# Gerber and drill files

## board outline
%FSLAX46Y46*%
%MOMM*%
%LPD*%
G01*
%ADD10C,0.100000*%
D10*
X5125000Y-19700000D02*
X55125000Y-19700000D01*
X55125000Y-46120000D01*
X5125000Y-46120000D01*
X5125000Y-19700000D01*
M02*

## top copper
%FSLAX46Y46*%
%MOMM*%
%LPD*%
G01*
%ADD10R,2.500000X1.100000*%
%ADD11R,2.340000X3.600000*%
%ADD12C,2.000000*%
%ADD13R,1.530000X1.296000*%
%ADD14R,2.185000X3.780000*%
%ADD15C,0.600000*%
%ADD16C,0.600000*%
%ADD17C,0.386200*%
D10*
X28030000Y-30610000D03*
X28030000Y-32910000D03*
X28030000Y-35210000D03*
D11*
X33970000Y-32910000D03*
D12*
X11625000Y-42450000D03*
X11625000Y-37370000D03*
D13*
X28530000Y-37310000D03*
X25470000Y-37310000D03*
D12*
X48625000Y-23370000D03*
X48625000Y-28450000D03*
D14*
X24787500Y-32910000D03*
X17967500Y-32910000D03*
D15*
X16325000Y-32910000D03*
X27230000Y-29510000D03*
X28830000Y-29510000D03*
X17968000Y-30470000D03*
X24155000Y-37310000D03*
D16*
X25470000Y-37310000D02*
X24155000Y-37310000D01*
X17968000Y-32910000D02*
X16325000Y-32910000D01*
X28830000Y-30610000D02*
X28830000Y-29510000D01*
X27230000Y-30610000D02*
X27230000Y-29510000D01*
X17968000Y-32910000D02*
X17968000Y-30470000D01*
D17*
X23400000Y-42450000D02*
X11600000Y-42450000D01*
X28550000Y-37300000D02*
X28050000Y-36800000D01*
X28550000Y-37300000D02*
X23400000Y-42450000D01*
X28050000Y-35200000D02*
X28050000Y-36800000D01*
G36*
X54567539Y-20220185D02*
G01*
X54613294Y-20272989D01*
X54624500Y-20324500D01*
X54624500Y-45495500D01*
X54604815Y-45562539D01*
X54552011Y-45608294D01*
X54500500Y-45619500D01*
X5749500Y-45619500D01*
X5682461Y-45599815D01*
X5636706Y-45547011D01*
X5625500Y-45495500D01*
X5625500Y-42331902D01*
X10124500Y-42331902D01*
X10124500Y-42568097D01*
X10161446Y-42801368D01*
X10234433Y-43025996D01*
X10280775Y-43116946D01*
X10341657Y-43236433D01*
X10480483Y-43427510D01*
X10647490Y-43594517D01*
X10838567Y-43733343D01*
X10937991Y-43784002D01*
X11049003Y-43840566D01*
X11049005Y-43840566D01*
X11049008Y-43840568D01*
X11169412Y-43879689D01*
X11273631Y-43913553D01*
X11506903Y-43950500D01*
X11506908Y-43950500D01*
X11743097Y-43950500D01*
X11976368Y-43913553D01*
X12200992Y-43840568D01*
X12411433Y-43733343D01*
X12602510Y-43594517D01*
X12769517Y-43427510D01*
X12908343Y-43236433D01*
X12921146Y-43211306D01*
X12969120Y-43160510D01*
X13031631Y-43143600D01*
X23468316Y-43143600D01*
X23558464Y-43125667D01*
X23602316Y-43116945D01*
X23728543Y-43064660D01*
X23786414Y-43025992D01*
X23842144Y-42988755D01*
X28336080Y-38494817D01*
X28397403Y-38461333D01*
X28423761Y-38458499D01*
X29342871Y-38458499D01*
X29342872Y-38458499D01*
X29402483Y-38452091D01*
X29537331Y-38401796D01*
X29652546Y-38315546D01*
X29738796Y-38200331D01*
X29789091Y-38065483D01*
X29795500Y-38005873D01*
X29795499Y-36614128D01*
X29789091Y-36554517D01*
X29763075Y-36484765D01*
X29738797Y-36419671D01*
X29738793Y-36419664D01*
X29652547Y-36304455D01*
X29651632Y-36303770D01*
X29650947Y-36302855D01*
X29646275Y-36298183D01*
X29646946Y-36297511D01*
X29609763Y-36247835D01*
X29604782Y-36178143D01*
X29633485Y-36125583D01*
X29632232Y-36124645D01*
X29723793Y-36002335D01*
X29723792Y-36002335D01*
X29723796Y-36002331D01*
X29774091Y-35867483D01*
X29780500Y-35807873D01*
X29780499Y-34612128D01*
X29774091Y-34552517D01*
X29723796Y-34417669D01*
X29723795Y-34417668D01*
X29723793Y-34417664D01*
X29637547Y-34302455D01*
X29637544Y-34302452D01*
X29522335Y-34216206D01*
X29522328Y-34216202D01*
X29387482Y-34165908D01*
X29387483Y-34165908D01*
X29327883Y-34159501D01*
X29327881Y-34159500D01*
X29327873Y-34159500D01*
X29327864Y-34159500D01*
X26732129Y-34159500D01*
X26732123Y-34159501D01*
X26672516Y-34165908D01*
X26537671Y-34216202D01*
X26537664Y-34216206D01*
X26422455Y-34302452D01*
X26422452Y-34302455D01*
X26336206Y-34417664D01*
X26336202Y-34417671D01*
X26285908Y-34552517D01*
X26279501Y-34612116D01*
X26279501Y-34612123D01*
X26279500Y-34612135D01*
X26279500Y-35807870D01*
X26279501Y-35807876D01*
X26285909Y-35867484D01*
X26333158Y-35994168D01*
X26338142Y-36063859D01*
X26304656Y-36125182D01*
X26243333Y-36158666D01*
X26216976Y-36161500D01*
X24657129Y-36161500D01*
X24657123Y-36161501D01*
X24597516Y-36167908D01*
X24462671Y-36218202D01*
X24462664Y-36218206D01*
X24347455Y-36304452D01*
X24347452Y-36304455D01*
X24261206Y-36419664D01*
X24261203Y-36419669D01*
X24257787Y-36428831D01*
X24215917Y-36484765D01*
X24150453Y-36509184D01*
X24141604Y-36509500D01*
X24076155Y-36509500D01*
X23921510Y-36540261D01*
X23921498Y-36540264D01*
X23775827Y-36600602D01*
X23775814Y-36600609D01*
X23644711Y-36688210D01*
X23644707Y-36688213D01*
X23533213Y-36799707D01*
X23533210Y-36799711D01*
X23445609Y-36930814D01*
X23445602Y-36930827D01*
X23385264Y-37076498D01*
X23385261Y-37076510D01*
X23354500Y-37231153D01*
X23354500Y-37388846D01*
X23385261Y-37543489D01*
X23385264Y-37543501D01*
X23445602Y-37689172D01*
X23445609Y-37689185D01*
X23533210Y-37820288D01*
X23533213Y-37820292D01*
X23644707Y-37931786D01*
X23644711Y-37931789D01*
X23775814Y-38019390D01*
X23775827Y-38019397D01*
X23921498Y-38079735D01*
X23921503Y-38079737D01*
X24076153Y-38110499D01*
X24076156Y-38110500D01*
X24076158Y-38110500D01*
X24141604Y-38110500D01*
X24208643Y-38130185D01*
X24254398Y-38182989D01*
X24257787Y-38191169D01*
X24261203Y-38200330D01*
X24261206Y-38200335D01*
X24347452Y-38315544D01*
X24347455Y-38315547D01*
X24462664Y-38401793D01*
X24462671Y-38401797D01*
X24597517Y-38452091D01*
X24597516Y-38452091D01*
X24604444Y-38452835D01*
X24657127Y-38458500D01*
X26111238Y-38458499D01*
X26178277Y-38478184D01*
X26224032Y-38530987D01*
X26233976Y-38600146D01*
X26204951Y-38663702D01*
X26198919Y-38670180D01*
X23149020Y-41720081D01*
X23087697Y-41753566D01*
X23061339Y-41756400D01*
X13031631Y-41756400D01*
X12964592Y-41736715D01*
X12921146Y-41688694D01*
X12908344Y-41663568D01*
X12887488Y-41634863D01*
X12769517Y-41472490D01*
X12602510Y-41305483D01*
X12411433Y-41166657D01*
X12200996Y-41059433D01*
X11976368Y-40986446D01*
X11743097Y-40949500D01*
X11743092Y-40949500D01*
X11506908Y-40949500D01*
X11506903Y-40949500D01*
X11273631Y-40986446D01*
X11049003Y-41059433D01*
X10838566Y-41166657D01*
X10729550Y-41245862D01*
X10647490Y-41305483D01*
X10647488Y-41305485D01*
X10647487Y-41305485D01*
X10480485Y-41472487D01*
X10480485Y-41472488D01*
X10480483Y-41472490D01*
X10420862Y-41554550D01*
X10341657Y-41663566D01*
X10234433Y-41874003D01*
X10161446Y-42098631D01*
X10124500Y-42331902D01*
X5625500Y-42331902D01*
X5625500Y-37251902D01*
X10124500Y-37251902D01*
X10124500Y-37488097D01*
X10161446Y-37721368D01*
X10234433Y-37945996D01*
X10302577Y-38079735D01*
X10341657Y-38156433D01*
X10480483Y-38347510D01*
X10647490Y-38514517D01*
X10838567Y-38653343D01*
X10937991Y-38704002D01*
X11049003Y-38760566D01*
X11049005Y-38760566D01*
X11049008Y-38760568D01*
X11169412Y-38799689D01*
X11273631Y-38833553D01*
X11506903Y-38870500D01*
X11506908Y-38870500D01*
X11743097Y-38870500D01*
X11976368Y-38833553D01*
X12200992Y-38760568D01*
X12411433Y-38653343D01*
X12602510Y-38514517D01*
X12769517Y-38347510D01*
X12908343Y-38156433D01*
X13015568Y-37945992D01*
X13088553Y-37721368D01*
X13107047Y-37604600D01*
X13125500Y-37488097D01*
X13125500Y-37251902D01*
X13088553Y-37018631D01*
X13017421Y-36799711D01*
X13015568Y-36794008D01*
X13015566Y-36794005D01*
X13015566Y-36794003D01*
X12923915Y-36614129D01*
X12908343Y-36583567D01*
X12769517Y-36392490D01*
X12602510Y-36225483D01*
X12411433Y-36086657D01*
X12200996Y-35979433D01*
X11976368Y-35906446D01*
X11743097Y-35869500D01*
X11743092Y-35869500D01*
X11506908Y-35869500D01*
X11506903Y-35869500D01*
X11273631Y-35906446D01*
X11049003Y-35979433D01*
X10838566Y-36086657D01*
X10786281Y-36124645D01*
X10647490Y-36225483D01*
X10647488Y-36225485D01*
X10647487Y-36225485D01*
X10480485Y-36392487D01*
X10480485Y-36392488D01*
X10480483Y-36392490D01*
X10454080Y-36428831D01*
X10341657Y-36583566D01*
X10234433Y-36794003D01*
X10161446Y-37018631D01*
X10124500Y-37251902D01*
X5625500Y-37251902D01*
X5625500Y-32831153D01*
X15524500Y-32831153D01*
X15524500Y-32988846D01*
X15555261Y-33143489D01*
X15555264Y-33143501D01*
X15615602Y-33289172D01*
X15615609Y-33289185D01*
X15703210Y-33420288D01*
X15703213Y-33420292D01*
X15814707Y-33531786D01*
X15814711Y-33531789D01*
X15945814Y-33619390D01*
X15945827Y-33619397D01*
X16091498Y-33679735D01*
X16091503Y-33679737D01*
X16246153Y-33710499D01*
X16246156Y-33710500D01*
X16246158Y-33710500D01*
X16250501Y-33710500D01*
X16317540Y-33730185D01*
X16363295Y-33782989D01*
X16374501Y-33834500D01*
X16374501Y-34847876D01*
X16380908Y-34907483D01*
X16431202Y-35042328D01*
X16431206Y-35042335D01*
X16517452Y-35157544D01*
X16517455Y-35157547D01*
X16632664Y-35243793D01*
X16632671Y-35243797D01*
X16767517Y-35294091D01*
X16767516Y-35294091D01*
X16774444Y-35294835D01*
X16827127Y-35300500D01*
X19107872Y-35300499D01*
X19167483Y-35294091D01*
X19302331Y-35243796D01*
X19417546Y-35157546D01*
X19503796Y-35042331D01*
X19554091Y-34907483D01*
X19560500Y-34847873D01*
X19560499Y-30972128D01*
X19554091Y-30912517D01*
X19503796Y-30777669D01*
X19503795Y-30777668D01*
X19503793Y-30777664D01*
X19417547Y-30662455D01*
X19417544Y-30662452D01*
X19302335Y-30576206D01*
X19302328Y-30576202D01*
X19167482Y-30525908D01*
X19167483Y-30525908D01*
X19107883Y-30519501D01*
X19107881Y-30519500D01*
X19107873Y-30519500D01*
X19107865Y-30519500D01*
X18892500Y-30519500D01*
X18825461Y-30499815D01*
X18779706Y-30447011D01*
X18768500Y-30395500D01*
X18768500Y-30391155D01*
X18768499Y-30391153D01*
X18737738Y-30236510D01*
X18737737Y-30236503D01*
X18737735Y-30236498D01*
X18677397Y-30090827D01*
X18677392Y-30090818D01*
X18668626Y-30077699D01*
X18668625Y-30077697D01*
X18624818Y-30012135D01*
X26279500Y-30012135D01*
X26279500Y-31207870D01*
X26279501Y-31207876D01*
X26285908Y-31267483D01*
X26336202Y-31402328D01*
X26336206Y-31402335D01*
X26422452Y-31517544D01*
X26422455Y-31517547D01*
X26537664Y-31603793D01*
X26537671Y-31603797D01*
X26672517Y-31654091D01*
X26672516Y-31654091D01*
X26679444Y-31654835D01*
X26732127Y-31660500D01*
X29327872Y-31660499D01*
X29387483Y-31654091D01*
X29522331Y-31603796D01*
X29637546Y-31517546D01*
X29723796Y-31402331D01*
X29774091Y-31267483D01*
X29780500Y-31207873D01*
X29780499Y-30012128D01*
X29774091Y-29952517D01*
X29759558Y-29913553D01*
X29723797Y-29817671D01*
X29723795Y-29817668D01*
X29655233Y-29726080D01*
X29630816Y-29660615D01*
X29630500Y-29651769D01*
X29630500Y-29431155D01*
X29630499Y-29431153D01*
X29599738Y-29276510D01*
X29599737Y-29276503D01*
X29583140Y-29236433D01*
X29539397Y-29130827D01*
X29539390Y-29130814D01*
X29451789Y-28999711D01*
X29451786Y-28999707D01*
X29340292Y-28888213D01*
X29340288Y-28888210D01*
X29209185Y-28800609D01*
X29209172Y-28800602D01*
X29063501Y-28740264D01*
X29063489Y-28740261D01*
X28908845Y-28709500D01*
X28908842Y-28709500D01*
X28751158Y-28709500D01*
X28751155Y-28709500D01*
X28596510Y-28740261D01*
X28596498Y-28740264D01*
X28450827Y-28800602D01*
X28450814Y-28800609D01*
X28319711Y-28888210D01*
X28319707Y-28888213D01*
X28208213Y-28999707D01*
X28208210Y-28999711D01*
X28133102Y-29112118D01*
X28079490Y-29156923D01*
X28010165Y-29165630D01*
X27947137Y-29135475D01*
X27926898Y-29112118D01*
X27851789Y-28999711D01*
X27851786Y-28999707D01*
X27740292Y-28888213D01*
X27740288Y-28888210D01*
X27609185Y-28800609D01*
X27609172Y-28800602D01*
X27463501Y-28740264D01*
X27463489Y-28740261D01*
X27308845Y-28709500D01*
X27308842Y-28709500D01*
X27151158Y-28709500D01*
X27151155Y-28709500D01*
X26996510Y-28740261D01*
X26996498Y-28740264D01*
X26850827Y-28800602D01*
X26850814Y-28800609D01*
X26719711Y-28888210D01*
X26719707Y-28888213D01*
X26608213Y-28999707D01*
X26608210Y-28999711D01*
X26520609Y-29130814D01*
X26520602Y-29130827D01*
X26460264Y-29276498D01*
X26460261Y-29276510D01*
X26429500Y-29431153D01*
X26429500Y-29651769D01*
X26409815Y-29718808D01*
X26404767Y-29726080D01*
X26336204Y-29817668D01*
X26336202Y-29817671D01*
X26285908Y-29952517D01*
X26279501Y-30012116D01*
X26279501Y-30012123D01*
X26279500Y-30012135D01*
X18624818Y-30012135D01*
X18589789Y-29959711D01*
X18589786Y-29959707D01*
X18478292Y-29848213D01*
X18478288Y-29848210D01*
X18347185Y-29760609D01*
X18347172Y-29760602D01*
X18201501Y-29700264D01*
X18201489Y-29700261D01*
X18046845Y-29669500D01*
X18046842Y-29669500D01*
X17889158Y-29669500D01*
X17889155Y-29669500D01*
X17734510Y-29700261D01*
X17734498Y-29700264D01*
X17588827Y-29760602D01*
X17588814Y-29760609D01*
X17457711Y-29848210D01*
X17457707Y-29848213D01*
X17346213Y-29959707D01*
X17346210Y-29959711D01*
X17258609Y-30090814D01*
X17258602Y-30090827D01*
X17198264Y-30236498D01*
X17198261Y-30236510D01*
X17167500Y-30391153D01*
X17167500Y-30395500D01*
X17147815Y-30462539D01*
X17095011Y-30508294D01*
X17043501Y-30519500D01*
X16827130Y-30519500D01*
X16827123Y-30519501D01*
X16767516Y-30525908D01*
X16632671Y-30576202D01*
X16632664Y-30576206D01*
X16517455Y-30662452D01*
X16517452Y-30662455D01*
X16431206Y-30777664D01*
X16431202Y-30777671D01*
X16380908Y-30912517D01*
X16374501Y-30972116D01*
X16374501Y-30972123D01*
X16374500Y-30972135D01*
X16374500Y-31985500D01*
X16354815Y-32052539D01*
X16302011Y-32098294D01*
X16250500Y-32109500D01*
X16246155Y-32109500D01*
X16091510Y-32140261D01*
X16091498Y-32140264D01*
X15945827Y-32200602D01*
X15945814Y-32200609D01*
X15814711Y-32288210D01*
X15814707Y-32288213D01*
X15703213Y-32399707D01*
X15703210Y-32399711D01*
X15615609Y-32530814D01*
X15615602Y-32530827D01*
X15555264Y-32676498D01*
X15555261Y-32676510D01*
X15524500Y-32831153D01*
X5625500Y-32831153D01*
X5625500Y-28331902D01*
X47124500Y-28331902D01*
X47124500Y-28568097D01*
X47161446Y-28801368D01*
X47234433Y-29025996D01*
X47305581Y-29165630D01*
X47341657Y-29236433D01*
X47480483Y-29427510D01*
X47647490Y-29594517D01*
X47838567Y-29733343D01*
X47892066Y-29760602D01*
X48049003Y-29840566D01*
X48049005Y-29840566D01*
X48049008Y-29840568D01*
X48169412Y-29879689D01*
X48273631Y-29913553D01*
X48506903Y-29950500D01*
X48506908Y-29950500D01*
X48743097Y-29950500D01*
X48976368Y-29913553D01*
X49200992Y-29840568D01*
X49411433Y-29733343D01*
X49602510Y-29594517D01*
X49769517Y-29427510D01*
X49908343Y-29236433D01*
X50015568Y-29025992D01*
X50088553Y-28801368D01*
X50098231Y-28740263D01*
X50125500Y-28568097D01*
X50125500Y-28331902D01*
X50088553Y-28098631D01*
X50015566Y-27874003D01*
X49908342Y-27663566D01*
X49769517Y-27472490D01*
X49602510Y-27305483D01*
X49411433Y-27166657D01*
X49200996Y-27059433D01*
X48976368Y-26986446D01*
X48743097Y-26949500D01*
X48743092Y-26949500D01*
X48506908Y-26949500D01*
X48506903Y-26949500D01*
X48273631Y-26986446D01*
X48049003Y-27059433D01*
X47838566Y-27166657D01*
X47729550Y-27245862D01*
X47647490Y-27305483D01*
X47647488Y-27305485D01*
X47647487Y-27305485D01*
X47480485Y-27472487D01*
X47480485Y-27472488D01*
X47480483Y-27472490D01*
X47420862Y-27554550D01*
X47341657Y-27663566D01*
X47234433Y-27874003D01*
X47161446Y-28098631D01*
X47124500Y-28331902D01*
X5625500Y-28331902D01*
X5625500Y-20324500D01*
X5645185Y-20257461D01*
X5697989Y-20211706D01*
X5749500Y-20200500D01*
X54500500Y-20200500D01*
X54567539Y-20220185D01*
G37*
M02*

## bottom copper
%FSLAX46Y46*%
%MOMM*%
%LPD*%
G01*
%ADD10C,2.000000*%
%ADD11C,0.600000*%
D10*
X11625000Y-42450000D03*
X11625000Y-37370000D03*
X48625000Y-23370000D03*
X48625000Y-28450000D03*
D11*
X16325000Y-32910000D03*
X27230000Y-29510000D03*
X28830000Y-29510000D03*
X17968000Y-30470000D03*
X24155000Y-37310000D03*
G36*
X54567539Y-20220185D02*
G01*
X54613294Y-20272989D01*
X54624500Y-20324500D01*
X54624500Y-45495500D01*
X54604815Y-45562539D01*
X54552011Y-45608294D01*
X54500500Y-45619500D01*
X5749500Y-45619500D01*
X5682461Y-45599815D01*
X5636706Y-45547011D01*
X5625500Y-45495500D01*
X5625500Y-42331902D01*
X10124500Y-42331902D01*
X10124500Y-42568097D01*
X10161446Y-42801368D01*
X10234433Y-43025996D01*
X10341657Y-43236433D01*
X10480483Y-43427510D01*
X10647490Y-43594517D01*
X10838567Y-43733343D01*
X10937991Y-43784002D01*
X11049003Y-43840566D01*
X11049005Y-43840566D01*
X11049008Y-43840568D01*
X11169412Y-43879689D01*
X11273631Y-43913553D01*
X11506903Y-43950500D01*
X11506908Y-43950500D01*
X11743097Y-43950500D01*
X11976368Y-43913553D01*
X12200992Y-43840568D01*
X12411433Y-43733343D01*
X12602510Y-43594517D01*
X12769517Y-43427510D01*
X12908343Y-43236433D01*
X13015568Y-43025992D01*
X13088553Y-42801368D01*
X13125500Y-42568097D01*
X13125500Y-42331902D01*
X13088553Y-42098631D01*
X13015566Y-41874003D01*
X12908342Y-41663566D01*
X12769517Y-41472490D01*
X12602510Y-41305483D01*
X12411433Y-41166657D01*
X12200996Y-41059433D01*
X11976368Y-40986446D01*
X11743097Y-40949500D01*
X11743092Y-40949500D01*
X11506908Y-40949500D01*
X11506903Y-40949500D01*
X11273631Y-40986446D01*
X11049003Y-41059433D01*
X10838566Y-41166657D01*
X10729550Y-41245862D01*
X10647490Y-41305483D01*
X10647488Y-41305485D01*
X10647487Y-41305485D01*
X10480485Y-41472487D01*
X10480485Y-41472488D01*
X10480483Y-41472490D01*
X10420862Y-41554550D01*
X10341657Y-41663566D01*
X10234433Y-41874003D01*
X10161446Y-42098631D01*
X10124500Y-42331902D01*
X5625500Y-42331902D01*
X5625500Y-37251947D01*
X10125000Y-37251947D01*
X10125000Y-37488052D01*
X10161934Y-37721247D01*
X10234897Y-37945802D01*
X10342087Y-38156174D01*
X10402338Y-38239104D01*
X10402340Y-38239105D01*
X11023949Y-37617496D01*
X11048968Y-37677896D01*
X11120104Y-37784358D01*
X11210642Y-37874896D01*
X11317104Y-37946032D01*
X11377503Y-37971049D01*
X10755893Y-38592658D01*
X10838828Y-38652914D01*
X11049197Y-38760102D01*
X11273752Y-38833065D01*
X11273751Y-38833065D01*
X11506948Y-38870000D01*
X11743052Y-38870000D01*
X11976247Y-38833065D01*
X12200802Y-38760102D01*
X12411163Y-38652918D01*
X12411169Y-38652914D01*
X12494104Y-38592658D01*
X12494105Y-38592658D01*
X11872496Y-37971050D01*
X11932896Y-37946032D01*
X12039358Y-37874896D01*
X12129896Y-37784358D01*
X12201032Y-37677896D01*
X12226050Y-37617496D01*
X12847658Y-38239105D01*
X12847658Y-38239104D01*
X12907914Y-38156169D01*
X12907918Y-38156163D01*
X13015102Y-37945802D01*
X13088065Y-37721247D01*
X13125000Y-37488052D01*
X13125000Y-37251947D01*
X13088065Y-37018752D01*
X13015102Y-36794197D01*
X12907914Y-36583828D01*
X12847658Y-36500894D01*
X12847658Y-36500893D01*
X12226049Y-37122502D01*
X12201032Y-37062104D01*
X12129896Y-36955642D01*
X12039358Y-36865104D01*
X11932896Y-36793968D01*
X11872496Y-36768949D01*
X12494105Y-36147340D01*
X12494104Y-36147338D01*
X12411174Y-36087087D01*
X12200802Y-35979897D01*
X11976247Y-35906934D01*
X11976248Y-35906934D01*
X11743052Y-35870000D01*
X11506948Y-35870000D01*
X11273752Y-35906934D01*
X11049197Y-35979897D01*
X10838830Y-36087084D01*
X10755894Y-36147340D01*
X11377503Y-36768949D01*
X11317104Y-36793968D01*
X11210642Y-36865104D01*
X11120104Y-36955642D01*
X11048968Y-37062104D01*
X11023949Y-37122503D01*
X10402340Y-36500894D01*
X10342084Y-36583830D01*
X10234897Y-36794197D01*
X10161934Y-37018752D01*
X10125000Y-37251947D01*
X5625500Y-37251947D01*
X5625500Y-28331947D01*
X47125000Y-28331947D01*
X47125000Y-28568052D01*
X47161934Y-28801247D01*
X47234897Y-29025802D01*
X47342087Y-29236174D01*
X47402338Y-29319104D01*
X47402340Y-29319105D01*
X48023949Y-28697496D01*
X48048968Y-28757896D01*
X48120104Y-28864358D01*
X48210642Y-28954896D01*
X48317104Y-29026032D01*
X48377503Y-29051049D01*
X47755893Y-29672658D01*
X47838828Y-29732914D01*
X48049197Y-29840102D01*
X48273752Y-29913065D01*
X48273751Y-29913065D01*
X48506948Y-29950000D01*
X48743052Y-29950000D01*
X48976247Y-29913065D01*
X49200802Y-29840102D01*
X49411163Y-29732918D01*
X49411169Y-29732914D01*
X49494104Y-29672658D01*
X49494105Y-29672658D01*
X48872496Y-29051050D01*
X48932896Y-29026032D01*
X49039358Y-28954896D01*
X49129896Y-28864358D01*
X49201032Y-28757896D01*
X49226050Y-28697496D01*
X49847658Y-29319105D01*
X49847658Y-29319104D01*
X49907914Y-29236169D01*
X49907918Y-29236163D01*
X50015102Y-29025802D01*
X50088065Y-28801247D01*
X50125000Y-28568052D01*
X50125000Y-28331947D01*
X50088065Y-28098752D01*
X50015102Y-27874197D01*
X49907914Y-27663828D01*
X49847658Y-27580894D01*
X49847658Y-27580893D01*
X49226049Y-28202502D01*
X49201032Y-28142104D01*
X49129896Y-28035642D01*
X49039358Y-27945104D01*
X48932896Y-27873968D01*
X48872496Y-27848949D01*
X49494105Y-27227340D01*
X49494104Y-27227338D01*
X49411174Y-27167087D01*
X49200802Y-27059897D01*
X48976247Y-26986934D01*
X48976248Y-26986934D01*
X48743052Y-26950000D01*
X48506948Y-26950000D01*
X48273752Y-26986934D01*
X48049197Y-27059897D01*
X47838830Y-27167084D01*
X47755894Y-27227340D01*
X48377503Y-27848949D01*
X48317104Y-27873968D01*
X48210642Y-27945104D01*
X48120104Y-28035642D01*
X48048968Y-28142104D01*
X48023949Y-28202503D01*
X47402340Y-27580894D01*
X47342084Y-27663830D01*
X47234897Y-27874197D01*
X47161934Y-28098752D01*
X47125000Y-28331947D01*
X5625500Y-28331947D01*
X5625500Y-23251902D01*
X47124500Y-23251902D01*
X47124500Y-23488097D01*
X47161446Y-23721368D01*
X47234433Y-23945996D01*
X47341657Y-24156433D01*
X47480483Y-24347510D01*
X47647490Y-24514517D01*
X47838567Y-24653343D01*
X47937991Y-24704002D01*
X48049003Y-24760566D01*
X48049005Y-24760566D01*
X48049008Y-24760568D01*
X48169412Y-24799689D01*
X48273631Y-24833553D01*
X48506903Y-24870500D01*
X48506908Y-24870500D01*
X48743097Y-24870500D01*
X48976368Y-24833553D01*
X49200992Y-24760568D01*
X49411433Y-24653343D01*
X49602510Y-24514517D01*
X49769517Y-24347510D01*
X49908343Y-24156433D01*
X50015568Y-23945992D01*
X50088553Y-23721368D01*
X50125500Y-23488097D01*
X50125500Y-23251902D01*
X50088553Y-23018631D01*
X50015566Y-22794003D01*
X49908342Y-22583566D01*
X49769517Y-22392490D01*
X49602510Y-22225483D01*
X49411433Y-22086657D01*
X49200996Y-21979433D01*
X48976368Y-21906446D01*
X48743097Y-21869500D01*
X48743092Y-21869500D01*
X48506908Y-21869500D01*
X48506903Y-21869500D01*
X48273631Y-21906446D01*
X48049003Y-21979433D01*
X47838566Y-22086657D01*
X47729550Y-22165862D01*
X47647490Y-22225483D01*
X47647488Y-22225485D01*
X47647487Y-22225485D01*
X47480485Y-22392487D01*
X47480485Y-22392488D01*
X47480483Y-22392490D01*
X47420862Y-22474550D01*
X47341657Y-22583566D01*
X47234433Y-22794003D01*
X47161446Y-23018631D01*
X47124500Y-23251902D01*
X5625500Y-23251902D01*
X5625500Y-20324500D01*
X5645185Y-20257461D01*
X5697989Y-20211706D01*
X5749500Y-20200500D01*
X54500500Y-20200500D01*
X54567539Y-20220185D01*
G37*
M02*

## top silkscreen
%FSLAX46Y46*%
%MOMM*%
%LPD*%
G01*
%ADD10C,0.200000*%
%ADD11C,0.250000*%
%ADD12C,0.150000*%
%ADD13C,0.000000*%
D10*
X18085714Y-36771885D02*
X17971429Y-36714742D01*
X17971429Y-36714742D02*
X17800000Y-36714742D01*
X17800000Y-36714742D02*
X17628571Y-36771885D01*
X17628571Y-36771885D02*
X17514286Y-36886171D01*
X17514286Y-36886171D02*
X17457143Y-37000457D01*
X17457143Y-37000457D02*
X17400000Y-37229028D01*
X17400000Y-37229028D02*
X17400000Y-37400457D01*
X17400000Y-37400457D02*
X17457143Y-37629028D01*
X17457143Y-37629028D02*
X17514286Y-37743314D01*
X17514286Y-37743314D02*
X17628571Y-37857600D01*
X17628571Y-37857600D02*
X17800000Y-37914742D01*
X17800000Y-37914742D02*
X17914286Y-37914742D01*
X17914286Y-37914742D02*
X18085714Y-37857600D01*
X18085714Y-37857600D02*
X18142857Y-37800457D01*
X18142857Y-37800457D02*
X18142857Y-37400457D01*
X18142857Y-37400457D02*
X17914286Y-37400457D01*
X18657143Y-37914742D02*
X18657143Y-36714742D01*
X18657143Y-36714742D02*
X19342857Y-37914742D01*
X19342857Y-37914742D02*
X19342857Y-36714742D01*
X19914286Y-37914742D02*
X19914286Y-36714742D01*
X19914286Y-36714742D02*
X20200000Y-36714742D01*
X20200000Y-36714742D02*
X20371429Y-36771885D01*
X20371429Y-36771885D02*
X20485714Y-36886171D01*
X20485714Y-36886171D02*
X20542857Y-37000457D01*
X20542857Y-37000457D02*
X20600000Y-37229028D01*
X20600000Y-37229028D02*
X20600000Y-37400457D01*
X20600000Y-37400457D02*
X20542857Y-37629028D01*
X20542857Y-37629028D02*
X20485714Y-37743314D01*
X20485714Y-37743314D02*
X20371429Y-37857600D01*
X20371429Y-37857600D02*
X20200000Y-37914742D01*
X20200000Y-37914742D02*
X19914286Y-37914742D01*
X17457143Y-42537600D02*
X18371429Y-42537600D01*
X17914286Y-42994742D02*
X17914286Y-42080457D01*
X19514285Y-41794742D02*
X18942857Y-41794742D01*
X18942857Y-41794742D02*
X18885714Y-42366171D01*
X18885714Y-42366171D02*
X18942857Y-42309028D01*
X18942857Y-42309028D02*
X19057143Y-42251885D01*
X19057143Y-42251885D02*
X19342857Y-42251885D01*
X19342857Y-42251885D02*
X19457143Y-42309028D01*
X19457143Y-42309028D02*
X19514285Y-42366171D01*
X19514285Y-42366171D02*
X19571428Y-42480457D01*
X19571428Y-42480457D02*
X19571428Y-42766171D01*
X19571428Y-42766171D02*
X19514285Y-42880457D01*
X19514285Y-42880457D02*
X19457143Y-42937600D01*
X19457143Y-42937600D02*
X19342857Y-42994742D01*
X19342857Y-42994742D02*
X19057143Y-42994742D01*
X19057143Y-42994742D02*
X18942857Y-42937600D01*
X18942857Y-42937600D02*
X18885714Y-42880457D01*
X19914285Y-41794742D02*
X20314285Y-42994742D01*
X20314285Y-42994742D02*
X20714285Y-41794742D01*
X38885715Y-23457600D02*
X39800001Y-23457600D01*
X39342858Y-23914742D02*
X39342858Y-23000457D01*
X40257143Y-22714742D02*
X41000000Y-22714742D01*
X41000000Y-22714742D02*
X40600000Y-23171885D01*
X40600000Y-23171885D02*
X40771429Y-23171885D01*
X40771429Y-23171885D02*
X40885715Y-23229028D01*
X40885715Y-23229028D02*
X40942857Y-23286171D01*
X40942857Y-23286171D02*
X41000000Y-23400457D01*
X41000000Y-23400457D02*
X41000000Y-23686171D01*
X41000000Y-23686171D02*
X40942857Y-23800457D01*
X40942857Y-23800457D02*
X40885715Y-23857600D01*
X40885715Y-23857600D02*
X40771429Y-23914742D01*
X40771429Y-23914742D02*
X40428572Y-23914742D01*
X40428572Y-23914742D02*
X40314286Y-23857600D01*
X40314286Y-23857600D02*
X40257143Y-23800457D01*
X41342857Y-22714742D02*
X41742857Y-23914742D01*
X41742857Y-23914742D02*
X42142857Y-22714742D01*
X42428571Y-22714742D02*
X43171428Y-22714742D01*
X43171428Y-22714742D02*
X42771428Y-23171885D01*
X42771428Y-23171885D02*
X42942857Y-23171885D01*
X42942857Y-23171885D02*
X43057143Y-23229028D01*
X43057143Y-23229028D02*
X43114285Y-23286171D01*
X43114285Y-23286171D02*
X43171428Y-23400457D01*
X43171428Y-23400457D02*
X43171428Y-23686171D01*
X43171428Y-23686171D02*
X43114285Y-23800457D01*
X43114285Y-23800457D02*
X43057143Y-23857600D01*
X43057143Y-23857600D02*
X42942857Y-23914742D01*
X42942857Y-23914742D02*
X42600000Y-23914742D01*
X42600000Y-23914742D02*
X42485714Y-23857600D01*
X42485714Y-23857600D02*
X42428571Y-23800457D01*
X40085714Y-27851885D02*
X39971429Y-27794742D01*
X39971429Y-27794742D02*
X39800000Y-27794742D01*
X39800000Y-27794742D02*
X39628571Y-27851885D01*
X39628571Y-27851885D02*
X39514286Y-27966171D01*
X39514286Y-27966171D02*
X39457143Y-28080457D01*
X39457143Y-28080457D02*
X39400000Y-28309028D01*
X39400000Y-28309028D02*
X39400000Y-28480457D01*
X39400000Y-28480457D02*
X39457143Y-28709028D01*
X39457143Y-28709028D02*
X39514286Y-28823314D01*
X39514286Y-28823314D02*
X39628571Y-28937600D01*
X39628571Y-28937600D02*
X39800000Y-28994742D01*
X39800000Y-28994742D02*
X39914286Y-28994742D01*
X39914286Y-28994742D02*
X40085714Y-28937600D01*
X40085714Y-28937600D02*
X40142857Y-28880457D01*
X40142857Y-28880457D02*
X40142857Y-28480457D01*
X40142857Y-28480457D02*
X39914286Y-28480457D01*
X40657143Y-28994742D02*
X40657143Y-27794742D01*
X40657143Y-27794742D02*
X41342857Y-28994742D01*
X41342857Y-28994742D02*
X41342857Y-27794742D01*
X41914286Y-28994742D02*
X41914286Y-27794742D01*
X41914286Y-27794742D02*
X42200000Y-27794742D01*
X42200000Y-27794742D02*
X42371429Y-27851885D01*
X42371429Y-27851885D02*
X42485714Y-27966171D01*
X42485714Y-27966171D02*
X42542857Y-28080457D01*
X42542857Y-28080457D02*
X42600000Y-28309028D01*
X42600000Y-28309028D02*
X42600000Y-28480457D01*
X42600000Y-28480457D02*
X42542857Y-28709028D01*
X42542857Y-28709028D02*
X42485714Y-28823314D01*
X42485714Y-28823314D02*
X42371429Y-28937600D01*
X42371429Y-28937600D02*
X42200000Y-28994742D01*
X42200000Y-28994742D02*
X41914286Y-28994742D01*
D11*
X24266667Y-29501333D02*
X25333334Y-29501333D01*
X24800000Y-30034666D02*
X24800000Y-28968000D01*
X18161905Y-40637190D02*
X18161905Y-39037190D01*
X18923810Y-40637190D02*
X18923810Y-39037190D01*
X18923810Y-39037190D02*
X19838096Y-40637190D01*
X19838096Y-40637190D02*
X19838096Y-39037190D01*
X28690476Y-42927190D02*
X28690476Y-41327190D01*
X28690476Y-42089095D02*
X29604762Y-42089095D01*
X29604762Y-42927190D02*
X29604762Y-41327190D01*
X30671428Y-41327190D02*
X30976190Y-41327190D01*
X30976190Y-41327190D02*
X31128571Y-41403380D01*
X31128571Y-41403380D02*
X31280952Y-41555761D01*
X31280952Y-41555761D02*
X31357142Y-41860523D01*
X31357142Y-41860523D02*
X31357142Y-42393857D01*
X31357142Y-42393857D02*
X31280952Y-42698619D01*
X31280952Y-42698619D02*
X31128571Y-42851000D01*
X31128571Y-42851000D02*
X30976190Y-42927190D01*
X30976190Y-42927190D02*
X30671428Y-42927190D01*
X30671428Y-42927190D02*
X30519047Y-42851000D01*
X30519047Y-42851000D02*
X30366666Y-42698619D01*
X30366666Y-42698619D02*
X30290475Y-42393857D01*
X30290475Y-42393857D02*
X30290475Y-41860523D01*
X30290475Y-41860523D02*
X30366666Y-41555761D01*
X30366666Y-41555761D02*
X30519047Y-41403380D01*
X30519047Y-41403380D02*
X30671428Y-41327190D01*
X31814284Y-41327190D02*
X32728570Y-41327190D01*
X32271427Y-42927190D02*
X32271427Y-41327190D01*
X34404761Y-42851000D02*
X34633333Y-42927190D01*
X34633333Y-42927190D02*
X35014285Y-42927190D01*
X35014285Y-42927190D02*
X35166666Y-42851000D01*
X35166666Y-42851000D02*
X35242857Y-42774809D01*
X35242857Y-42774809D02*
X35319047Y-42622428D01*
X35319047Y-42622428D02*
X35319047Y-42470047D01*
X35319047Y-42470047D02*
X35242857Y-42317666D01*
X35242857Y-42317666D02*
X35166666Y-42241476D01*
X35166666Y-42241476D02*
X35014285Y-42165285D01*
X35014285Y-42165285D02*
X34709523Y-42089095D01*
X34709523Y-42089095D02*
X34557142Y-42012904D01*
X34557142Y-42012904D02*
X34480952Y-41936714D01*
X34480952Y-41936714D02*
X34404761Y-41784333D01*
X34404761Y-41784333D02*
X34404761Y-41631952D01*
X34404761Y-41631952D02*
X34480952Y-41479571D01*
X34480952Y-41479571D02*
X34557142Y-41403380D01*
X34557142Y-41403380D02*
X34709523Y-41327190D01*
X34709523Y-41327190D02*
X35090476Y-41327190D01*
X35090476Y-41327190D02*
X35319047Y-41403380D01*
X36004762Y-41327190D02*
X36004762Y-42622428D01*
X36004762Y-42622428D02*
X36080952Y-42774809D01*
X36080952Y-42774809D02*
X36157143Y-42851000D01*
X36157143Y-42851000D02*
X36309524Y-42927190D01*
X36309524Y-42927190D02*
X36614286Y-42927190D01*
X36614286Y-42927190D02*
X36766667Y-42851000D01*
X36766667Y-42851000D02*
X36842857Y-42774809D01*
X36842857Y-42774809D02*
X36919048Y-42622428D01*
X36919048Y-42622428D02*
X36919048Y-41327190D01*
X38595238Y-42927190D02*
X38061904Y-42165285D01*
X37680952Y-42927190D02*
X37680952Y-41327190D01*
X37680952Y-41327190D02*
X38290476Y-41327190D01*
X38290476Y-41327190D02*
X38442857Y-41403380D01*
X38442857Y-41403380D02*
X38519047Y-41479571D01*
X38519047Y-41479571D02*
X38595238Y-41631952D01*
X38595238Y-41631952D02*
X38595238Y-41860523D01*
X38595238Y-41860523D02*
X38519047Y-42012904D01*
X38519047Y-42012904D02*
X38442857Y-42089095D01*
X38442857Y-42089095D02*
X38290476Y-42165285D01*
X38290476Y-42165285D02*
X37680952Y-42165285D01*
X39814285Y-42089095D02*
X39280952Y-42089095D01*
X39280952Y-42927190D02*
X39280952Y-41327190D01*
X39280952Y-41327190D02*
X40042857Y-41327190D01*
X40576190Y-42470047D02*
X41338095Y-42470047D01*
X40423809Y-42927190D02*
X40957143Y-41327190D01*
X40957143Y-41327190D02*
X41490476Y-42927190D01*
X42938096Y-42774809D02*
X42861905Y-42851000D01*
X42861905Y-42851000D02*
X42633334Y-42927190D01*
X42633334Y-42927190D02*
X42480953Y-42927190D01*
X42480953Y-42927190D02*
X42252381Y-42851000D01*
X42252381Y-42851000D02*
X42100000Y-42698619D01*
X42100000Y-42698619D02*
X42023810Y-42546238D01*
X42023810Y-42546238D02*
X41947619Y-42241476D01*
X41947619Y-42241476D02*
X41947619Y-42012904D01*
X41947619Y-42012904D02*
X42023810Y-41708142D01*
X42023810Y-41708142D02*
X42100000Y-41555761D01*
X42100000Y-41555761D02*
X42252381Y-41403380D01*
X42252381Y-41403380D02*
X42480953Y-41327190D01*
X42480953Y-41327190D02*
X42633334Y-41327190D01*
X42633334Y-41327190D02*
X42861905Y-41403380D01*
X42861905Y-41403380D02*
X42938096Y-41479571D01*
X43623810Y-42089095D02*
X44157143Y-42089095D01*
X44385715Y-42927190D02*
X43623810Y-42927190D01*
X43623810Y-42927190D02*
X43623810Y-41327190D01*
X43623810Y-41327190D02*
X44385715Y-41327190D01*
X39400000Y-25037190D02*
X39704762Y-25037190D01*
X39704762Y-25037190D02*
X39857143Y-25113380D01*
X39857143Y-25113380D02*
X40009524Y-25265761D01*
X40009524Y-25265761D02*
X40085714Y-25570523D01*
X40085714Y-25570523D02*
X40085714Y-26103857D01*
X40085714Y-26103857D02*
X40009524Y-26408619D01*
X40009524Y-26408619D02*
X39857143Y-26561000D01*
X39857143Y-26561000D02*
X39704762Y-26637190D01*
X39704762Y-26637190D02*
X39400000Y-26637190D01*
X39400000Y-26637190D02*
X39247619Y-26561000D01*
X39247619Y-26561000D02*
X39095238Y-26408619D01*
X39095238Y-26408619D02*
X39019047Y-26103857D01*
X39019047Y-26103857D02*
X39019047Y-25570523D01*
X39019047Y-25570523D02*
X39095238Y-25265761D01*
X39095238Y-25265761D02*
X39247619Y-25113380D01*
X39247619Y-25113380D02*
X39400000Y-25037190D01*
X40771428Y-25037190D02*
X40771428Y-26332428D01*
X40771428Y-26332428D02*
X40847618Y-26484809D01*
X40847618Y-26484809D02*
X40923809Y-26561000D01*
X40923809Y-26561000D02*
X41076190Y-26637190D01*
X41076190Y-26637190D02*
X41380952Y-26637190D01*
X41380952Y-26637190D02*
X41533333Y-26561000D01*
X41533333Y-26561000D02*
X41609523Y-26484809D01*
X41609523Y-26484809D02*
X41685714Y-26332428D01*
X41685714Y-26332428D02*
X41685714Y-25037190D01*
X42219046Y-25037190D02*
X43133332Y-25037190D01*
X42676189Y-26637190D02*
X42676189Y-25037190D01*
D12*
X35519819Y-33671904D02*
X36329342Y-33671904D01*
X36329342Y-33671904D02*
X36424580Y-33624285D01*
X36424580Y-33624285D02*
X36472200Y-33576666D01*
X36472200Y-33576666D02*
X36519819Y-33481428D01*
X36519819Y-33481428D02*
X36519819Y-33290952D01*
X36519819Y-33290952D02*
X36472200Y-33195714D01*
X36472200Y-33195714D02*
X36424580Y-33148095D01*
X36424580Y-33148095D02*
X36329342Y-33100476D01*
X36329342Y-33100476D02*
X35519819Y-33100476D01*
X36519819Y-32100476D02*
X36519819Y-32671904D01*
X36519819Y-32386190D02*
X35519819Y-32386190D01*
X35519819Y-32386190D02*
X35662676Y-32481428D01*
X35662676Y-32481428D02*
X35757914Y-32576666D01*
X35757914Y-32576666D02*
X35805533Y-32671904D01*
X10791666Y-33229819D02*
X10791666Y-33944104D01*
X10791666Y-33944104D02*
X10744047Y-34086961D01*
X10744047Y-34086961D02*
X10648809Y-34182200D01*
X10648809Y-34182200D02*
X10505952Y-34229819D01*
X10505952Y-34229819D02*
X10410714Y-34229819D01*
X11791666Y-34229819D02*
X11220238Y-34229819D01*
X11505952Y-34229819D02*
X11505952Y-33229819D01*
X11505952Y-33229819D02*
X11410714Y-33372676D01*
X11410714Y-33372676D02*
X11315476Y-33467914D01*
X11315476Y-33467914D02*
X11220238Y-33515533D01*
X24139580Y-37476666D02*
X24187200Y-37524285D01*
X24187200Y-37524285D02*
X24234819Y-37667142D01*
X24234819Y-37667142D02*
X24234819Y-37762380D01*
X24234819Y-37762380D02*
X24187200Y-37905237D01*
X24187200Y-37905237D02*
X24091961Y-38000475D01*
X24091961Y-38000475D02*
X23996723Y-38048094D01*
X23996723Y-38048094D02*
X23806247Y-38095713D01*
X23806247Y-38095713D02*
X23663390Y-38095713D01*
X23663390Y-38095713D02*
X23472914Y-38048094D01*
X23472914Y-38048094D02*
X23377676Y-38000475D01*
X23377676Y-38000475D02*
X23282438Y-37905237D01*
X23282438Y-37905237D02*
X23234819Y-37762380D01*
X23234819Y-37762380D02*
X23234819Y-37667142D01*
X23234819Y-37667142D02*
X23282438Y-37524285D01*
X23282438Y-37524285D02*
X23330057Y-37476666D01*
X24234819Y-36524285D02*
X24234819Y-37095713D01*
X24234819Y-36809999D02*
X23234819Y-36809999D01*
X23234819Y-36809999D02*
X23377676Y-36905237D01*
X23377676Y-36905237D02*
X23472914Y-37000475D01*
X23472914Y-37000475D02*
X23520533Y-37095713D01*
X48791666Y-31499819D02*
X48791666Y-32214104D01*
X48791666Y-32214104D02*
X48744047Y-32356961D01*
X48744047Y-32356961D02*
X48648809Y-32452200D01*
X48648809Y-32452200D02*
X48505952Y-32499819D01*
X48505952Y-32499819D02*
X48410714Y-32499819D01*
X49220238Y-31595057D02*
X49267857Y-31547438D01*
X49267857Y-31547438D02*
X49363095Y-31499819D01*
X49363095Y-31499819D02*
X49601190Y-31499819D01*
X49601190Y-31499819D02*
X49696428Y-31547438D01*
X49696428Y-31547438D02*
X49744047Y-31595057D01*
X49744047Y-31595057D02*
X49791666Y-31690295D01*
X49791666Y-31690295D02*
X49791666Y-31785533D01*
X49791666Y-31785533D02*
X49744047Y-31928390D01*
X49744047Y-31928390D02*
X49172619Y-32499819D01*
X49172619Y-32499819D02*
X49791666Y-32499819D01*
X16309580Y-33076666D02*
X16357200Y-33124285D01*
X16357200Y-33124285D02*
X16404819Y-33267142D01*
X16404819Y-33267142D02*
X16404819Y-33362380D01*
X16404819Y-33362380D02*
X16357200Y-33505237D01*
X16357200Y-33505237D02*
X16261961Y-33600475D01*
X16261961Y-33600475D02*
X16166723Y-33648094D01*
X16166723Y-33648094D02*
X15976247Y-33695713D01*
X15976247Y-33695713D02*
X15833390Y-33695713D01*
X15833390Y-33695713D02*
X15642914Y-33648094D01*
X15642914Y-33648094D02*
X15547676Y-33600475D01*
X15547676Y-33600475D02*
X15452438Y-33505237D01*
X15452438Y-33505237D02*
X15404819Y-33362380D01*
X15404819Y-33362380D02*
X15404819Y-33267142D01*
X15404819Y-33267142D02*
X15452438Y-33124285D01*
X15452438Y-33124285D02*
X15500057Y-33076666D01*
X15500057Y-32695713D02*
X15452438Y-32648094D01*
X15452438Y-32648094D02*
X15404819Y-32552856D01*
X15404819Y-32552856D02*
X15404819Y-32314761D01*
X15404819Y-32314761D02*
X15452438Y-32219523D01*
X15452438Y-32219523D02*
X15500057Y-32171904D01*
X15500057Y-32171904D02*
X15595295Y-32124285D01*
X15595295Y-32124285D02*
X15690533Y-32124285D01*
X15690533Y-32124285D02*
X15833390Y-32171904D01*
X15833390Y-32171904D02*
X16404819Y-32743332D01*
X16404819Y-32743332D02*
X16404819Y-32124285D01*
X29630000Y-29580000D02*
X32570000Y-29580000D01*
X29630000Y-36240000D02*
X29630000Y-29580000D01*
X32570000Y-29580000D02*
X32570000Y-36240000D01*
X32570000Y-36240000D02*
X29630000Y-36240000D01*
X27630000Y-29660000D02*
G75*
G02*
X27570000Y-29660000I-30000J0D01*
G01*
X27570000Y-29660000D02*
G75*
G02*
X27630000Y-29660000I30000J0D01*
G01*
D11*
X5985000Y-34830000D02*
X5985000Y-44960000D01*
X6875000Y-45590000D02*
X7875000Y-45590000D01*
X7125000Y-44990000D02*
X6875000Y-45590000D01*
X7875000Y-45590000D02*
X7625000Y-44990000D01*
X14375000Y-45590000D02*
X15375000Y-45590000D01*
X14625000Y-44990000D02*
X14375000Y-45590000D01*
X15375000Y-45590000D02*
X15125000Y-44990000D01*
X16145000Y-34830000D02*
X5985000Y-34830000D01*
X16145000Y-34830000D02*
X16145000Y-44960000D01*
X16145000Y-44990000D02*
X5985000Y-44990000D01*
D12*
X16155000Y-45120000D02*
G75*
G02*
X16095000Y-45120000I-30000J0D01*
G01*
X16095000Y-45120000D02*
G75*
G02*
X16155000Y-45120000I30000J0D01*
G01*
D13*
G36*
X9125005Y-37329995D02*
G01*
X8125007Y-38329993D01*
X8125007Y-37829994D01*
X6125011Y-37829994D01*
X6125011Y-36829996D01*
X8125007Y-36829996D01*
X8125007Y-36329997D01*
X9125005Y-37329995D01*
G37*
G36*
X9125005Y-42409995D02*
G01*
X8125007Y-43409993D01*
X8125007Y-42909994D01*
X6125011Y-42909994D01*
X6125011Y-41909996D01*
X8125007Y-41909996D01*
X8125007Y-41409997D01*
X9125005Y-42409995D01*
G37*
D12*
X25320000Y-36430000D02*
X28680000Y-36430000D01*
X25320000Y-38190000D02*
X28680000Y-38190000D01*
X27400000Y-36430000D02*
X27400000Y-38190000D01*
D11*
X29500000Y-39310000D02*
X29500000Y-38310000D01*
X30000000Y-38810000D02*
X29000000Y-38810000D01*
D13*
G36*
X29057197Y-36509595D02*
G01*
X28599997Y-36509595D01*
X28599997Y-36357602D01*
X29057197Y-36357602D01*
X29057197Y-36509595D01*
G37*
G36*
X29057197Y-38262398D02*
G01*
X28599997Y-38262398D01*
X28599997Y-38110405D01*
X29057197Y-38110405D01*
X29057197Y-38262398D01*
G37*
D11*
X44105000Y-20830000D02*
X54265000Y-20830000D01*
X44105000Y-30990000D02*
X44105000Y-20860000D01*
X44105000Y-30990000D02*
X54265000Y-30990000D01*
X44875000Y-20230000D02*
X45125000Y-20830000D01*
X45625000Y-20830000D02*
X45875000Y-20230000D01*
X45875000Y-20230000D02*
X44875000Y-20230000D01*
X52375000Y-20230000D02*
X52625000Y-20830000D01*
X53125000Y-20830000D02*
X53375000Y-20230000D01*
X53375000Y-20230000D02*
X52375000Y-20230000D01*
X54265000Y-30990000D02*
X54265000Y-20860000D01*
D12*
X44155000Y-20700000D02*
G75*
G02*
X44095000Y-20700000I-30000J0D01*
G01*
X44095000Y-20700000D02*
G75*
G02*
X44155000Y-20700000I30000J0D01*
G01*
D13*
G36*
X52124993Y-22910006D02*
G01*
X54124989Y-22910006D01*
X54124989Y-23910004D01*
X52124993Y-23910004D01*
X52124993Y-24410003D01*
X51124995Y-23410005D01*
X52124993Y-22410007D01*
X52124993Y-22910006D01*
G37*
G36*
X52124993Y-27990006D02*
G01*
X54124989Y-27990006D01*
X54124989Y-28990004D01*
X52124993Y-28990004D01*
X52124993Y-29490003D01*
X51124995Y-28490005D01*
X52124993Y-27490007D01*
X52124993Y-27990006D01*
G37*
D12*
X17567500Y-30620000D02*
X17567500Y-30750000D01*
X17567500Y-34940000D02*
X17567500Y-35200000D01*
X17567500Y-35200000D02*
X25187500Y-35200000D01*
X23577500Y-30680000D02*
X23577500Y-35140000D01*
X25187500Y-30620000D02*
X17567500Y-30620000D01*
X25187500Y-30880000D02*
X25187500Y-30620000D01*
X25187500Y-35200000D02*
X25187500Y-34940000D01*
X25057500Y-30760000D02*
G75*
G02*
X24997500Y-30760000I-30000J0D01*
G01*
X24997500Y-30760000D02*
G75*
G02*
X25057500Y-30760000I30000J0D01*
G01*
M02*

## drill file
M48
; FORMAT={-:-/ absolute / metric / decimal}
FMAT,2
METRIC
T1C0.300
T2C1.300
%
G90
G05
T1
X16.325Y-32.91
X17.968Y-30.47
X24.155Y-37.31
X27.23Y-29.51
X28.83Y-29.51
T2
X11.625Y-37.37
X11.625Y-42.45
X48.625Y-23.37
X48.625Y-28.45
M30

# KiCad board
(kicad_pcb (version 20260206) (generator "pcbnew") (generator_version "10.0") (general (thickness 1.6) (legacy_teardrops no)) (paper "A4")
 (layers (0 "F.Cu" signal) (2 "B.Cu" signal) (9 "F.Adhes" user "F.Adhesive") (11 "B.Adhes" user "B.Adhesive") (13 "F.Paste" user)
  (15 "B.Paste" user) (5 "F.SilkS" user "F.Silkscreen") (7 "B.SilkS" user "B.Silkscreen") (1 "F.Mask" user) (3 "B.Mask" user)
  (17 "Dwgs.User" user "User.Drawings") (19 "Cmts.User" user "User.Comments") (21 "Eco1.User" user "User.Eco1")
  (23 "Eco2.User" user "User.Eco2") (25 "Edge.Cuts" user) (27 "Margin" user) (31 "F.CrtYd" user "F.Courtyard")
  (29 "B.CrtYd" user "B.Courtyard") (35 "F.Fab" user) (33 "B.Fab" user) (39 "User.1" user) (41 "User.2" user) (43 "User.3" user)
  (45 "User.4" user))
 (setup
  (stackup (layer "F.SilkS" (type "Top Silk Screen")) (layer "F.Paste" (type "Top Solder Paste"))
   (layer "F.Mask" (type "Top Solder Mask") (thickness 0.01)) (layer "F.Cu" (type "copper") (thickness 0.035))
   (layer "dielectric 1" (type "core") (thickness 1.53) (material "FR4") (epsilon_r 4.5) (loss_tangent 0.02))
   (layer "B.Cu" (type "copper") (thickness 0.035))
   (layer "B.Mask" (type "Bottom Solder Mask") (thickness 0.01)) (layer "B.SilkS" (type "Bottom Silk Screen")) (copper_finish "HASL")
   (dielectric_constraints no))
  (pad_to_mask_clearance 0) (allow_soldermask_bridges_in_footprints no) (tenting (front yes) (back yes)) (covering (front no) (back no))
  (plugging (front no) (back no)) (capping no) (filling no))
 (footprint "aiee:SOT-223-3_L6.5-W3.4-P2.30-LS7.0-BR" (layer "F.Cu") (at 31 32.91 180)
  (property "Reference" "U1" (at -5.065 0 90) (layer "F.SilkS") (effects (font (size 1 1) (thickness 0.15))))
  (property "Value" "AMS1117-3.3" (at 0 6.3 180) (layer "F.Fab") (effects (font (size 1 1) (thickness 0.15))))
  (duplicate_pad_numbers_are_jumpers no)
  (fp_line (start 1.37 3.33) (end -1.57 3.33) (stroke (width 0.15) (type solid)) (layer "F.SilkS"))
  (fp_line (start 1.37 -3.33) (end 1.37 3.33) (stroke (width 0.15) (type solid)) (layer "F.SilkS"))
  (fp_line (start -1.57 3.33) (end -1.57 -3.33) (stroke (width 0.15) (type solid)) (layer "F.SilkS"))
  (fp_line (start -1.57 -3.33) (end 1.37 -3.33) (stroke (width 0.15) (type solid)) (layer "F.SilkS"))
  (fp_circle (center 3.4 3.25) (end 3.43 3.25) (stroke (width 0.15) (type solid)) (fill no) (layer "F.SilkS"))
  (pad "1" smd rect (at 2.97 2.3 180) (size 2.5 1.1) (layers "F.Cu" "F.Mask" "F.Paste") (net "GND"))
  (pad "2" smd rect (at 2.97 0 180) (size 2.5 1.1) (layers "F.Cu" "F.Mask" "F.Paste") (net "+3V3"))
  (pad "3" smd rect (at 2.97 -2.3 180) (size 2.5 1.1) (layers "F.Cu" "F.Mask" "F.Paste") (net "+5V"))
  (pad "4" smd rect (at -2.97 0 180) (size 2.34 3.6) (layers "F.Cu" "F.Mask" "F.Paste") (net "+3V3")))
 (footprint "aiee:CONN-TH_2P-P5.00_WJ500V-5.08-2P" (layer "F.Cu") (at 11.625 39.91 90)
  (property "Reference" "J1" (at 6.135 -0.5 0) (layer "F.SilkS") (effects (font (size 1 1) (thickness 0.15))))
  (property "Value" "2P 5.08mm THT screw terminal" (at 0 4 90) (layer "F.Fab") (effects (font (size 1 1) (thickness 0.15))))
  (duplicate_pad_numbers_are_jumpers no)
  (fp_line (start 5.08 -5.64) (end -5.05 -5.64) (stroke (width 0.25) (type solid)) (layer "F.SilkS"))
  (fp_line (start -5.68 -4.75) (end -5.68 -3.75) (stroke (width 0.25) (type solid)) (layer "F.SilkS"))
  (fp_line (start -5.08 -4.5) (end -5.68 -4.75) (stroke (width 0.25) (type solid)) (layer "F.SilkS"))
  (fp_line (start -5.68 -3.75) (end -5.08 -4) (stroke (width 0.25) (type solid)) (layer "F.SilkS"))
  (fp_line (start -5.68 2.75) (end -5.68 3.75) (stroke (width 0.25) (type solid)) (layer "F.SilkS"))
  (fp_line (start -5.08 3) (end -5.68 2.75) (stroke (width 0.25) (type solid)) (layer "F.SilkS"))
  (fp_line (start -5.68 3.75) (end -5.08 3.5) (stroke (width 0.25) (type solid)) (layer "F.SilkS"))
  (fp_line (start 5.08 4.52) (end 5.08 -5.64) (stroke (width 0.25) (type solid)) (layer "F.SilkS"))
  (fp_line (start 5.08 4.52) (end -5.05 4.52) (stroke (width 0.25) (type solid)) (layer "F.SilkS"))
  (fp_line (start -5.08 4.52) (end -5.08 -5.64) (stroke (width 0.25) (type solid)) (layer "F.SilkS"))
  (fp_circle (center -5.21 4.5) (end -5.18 4.5) (stroke (width 0.15) (type solid)) (fill no) (layer "F.SilkS"))
  (fp_poly
   (pts (xy 2.080006 -5.499989) (xy 3.080004 -5.499989) (xy 3.080004 -3.499993) (xy 3.580003 -3.499993) (xy 2.580005 -2.499995)
    (xy 1.580007 -3.499993) (xy 2.080006 -3.499993) (xy 2.080006 -5.499989))
   (stroke (width 0) (type solid)) (fill yes) (layer "F.SilkS"))
  (fp_poly
   (pts (xy -2.999994 -5.499989) (xy -1.999996 -5.499989) (xy -1.999996 -3.499993) (xy -1.499997 -3.499993) (xy -2.499995 -2.499995)
    (xy -3.499993 -3.499993) (xy -2.999994 -3.499993) (xy -2.999994 -5.499989))
   (stroke (width 0) (type solid)) (fill yes) (layer "F.SilkS"))
  (pad "1" thru_hole circle (at -2.54 0 270) (size 2 2) (drill 1.300022) (layers "*.Cu" "*.Mask") (remove_unused_layers no) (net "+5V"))
  (pad "2" thru_hole circle (at 2.54 0 270) (size 2 2) (drill 1.300022) (layers "*.Cu" "*.Mask") (remove_unused_layers no) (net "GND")))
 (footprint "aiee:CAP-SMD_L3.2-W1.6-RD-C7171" (layer "F.Cu") (at 27 37.31 180)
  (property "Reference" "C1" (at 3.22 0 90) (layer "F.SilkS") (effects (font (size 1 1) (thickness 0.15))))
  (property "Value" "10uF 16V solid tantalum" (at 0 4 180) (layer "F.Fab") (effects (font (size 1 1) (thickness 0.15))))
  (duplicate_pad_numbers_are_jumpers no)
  (fp_line (start 1.68 0.88) (end -1.68 0.88) (stroke (width 0.15) (type solid)) (layer "F.SilkS"))
  (fp_line (start 1.68 -0.88) (end -1.68 -0.88) (stroke (width 0.15) (type solid)) (layer "F.SilkS"))
  (fp_line (start -0.4 0.88) (end -0.4 -0.88) (stroke (width 0.15) (type solid)) (layer "F.SilkS"))
  (fp_line (start -2.5 -2) (end -2.5 -1) (stroke (width 0.25) (type solid)) (layer "F.SilkS"))
  (fp_line (start -3 -1.5) (end -2 -1.5) (stroke (width 0.25) (type solid)) (layer "F.SilkS"))
  (fp_poly
   (pts (xy -1.599997 0.952398) (xy -1.599997 0.800405) (xy -2.057197 0.800405) (xy -2.057197 0.952398) (xy -1.599997 0.952398))
   (stroke (width 0) (type solid)) (fill yes) (layer "F.SilkS"))
  (fp_poly
   (pts (xy -1.599997 -0.952398) (xy -1.599997 -0.800405) (xy -2.057197 -0.800405) (xy -2.057197 -0.952398) (xy -1.599997 -0.952398))
   (stroke (width 0) (type solid)) (fill yes) (layer "F.SilkS"))
  (pad "1" smd rect (at -1.53 0) (size 1.53 1.296) (layers "F.Cu" "F.Mask" "F.Paste") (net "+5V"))
  (pad "2" smd rect (at 1.53 0) (size 1.53 1.296) (layers "F.Cu" "F.Mask" "F.Paste") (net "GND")))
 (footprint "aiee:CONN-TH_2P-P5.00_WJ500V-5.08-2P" (layer "F.Cu") (at 48.625 25.91 -90)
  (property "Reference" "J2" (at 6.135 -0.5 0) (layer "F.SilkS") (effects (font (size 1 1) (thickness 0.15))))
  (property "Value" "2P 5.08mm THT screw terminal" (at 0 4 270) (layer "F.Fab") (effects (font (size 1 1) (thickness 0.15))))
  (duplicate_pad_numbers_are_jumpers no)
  (fp_line (start -5.08 4.52) (end -5.08 -5.64) (stroke (width 0.25) (type solid)) (layer "F.SilkS"))
  (fp_line (start 5.08 4.52) (end -5.05 4.52) (stroke (width 0.25) (type solid)) (layer "F.SilkS"))
  (fp_line (start 5.08 4.52) (end 5.08 -5.64) (stroke (width 0.25) (type solid)) (layer "F.SilkS"))
  (fp_line (start -5.68 3.75) (end -5.08 3.5) (stroke (width 0.25) (type solid)) (layer "F.SilkS"))
  (fp_line (start -5.08 3) (end -5.68 2.75) (stroke (width 0.25) (type solid)) (layer "F.SilkS"))
  (fp_line (start -5.68 2.75) (end -5.68 3.75) (stroke (width 0.25) (type solid)) (layer "F.SilkS"))
  (fp_line (start -5.68 -3.75) (end -5.08 -4) (stroke (width 0.25) (type solid)) (layer "F.SilkS"))
  (fp_line (start -5.08 -4.5) (end -5.68 -4.75) (stroke (width 0.25) (type solid)) (layer "F.SilkS"))
  (fp_line (start -5.68 -4.75) (end -5.68 -3.75) (stroke (width 0.25) (type solid)) (layer "F.SilkS"))
  (fp_line (start 5.08 -5.64) (end -5.05 -5.64) (stroke (width 0.25) (type solid)) (layer "F.SilkS"))
  (fp_circle (center -5.21 4.5) (end -5.18 4.5) (stroke (width 0.15) (type solid)) (fill no) (layer "F.SilkS"))
  (fp_poly
   (pts (xy -2.999994 -5.499989) (xy -1.999996 -5.499989) (xy -1.999996 -3.499993) (xy -1.499997 -3.499993) (xy -2.499995 -2.499995)
    (xy -3.499993 -3.499993) (xy -2.999994 -3.499993) (xy -2.999994 -5.499989))
   (stroke (width 0) (type solid)) (fill yes) (layer "F.SilkS"))
  (fp_poly
   (pts (xy 2.080006 -5.499989) (xy 3.080004 -5.499989) (xy 3.080004 -3.499993) (xy 3.580003 -3.499993) (xy 2.580005 -2.499995)
    (xy 1.580007 -3.499993) (xy 2.080006 -3.499993) (xy 2.080006 -5.499989))
   (stroke (width 0) (type solid)) (fill yes) (layer "F.SilkS"))
  (pad "1" thru_hole circle (at -2.54 0 90) (size 2 2) (drill 1.300022) (layers "*.Cu" "*.Mask") (remove_unused_layers no) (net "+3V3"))
  (pad "2" thru_hole circle (at 2.54 0 90) (size 2 2) (drill 1.300022) (layers "*.Cu" "*.Mask") (remove_unused_layers no) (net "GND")))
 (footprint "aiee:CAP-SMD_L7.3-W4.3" (layer "F.Cu") (at 21.3775 32.91)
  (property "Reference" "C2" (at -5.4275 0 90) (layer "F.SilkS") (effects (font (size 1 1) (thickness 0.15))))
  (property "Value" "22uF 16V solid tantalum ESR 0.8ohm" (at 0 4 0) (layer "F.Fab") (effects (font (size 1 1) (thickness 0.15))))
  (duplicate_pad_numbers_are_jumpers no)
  (fp_line (start -3.81 -2.29) (end -3.81 -2.16) (stroke (width 0.15) (type solid)) (layer "F.SilkS"))
  (fp_line (start -3.81 2.03) (end -3.81 2.29) (stroke (width 0.15) (type solid)) (layer "F.SilkS"))
  (fp_line (start -3.81 2.29) (end 3.81 2.29) (stroke (width 0.15) (type solid)) (layer "F.SilkS"))
  (fp_line (start 2.2 -2.23) (end 2.2 2.23) (stroke (width 0.15) (type solid)) (layer "F.SilkS"))
  (fp_line (start 3.81 -2.29) (end -3.81 -2.29) (stroke (width 0.15) (type solid)) (layer "F.SilkS"))
  (fp_line (start 3.81 -2.03) (end 3.81 -2.29) (stroke (width 0.15) (type solid)) (layer "F.SilkS"))
  (fp_line (start 3.81 2.29) (end 3.81 2.03) (stroke (width 0.15) (type solid)) (layer "F.SilkS"))
  (fp_circle (center 3.65 -2.15) (end 3.68 -2.15) (stroke (width 0.15) (type solid)) (fill no) (layer "F.SilkS"))
  (pad "1" smd rect (at 3.41 0 180) (size 2.185 3.78) (layers "F.Cu" "F.Mask" "F.Paste") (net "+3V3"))
  (pad "2" smd rect (at -3.41 0 180) (size 2.185 3.78) (layers "F.Cu" "F.Mask" "F.Paste") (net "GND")))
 (gr_rect (start 5.125 19.7) (end 55.125 46.12) (stroke (width 0.1) (type default)) (fill no) (layer "Edge.Cuts"))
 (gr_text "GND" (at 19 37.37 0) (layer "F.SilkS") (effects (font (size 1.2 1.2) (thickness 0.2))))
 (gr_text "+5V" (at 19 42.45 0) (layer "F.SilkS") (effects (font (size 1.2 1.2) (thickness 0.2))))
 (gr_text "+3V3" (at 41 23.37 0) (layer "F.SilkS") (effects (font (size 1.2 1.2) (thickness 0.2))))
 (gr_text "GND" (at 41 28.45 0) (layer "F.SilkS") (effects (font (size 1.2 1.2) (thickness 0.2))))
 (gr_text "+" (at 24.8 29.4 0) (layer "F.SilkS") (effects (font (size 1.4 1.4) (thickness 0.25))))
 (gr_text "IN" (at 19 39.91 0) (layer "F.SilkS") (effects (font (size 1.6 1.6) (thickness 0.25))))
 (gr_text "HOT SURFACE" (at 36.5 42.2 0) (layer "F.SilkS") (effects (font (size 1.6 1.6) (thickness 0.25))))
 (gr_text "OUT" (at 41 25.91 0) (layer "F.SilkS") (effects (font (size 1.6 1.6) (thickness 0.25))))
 (segment (start 25.47 37.31) (end 24.155 37.31) (width 0.6) (layer "F.Cu") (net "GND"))
 (segment (start 17.968 32.91) (end 16.325 32.91) (width 0.6) (layer "F.Cu") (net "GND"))
 (segment (start 28.83 30.61) (end 28.83 29.51) (width 0.6) (layer "F.Cu") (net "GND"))
 (segment (start 27.23 30.61) (end 27.23 29.51) (width 0.6) (layer "F.Cu") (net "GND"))
 (segment (start 17.968 32.91) (end 17.968 30.47) (width 0.6) (layer "F.Cu") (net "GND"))
 (via (at 16.325 32.91) (size 0.6) (drill 0.3) (layers "F.Cu" "B.Cu") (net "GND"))
 (via (at 27.23 29.51) (size 0.6) (drill 0.3) (layers "F.Cu" "B.Cu") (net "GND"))
 (via (at 28.83 29.51) (size 0.6) (drill 0.3) (layers "F.Cu" "B.Cu") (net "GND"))
 (via (at 17.968 30.47) (size 0.6) (drill 0.3) (layers "F.Cu" "B.Cu") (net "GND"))
 (via (at 24.155 37.31) (size 0.6) (drill 0.3) (layers "F.Cu" "B.Cu") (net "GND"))
 (segment (start 23.4 42.45) (end 11.6 42.45) (width 0.3862) (layer "F.Cu") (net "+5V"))
 (segment (start 28.55 37.3) (end 28.05 36.8) (width 0.3862) (layer "F.Cu") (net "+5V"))
 (segment (start 28.55 37.3) (end 23.4 42.45) (width 0.3862) (layer "F.Cu") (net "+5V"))
 (segment (start 28.05 35.2) (end 28.05 36.8) (width 0.3862) (layer "F.Cu") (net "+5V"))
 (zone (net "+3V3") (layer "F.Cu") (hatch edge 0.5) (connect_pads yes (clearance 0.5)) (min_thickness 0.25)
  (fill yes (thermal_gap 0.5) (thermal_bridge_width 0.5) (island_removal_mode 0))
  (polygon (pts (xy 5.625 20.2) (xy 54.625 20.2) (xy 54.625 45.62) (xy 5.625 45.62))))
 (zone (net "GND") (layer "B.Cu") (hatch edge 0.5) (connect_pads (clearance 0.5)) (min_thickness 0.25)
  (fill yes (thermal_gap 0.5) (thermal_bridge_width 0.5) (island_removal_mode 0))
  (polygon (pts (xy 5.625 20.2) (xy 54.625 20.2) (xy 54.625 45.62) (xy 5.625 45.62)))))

